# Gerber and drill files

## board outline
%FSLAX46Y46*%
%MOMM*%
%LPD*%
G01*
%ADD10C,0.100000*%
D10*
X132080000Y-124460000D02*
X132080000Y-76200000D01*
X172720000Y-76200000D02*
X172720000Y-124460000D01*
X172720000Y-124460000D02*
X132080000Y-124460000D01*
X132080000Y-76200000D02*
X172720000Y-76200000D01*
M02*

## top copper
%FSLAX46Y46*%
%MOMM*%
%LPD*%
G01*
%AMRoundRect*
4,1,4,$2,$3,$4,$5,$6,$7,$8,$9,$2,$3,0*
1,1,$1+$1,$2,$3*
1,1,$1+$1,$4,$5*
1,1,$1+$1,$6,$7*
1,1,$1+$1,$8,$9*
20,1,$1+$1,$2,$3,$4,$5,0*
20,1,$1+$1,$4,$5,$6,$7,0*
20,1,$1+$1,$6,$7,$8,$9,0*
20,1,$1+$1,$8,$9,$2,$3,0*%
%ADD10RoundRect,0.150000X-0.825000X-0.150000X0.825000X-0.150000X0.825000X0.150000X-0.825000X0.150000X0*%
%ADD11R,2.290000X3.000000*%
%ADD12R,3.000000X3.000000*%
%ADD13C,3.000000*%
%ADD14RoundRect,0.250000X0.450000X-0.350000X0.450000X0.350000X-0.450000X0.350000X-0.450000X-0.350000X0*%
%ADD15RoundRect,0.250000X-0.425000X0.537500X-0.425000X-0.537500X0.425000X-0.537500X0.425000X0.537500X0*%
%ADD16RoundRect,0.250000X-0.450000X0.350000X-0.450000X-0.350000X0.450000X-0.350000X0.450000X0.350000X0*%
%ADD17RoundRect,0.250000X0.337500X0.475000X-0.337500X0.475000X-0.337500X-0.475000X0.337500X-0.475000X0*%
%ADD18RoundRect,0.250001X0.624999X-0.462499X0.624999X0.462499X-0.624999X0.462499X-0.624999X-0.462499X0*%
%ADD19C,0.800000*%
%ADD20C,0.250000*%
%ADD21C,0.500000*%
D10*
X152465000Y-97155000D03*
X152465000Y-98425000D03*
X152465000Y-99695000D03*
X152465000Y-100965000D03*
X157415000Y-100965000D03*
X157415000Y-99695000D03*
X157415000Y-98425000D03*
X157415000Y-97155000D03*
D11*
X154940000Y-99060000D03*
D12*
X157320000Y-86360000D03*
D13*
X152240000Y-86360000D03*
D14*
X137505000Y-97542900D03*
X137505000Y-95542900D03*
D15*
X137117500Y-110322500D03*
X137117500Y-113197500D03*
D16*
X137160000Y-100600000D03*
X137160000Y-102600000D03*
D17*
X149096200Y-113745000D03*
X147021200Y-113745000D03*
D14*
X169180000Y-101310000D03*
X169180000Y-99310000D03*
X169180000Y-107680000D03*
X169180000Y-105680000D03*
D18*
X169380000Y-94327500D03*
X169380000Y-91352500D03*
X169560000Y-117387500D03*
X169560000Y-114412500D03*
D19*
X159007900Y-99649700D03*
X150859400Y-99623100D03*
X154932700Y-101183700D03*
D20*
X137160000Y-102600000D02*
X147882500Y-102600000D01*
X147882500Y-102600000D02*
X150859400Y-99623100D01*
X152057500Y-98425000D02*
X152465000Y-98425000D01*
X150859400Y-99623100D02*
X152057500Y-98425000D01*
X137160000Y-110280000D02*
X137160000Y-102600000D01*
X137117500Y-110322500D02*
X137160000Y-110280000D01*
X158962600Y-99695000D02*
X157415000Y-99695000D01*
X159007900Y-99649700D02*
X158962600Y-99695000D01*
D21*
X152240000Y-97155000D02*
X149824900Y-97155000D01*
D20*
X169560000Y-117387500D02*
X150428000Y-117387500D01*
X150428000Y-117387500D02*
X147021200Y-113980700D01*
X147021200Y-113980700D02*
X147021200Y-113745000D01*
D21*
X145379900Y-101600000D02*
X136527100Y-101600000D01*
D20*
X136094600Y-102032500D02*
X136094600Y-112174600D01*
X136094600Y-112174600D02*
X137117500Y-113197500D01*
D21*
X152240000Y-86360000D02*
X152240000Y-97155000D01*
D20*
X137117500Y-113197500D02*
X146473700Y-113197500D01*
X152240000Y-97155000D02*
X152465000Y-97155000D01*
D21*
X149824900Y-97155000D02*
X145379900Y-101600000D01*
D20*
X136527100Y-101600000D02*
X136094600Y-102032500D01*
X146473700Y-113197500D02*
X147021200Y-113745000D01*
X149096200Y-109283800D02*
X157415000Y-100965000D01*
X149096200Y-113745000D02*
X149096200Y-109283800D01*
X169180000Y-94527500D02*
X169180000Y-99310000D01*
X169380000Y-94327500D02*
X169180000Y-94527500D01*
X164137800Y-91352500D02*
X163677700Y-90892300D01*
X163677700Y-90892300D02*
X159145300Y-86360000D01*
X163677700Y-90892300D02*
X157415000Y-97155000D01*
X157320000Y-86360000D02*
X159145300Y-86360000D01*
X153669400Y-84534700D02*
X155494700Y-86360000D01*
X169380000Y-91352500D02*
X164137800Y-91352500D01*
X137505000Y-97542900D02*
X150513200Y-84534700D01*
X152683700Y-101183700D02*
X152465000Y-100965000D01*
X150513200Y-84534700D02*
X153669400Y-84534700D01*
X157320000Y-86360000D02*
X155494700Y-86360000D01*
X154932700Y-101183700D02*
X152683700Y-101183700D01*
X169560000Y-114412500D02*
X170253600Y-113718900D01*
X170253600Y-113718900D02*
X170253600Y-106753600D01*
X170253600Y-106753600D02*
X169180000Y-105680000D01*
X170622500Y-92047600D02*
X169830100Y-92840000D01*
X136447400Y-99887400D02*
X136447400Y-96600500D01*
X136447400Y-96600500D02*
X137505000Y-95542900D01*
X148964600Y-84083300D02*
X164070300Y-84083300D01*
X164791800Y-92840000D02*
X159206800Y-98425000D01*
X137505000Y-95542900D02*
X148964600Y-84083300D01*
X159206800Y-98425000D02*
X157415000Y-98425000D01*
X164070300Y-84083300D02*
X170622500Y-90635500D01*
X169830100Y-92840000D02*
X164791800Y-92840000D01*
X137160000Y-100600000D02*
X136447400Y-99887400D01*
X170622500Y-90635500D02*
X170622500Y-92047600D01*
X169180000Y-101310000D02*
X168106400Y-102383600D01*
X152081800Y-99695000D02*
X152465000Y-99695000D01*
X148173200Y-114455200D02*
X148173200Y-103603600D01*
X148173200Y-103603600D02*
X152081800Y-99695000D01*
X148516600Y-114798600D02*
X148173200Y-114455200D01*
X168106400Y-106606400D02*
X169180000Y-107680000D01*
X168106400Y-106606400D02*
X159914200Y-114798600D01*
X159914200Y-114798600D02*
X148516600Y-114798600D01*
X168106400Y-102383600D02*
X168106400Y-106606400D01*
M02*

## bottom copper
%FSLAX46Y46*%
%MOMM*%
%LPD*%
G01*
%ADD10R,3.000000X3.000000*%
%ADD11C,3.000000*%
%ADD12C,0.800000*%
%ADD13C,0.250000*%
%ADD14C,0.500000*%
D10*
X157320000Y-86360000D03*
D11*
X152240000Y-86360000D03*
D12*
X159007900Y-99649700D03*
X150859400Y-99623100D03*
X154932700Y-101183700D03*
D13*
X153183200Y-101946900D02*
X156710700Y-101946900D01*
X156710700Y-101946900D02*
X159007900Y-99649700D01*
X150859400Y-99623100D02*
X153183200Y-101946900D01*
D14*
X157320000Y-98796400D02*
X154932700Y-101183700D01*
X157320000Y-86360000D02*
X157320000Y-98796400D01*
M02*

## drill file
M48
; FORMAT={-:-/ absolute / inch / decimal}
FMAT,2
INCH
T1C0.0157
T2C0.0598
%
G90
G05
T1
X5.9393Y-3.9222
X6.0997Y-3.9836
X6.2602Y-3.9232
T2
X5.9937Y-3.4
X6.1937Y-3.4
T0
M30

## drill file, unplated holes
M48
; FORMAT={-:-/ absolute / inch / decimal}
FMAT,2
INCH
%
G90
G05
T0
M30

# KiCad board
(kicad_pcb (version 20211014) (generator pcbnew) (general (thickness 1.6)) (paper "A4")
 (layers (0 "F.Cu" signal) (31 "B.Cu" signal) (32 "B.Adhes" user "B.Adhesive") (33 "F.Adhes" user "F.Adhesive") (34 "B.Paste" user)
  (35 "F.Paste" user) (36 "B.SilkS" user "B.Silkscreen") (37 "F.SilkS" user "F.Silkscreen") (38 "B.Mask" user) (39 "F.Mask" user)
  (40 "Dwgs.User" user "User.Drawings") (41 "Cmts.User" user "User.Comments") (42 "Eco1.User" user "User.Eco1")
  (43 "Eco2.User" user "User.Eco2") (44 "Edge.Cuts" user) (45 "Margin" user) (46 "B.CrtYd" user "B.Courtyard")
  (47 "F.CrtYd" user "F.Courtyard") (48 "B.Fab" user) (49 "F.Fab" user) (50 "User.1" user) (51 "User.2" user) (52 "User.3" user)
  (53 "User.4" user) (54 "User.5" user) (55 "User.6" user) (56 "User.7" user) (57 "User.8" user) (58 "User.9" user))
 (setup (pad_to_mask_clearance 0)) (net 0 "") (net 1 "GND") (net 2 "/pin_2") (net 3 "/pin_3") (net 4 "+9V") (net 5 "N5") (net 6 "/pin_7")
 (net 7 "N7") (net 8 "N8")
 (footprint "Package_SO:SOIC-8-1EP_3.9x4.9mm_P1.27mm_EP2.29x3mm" (layer "F.Cu") (at 154.94 99.06)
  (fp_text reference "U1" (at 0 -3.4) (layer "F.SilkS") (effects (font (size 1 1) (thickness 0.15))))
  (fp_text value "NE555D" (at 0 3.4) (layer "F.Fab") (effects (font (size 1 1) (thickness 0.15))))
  (pad "" smd roundrect (at 0.57 -0.75) (size 0.92 1.21) (layers "F.Paste") (roundrect_rratio 0.25))
  (pad "" smd roundrect (at -0.57 0.75) (size 0.92 1.21) (layers "F.Paste") (roundrect_rratio 0.25))
  (pad "" smd roundrect (at -0.57 -0.75) (size 0.92 1.21) (layers "F.Paste") (roundrect_rratio 0.25))
  (pad "" smd roundrect (at 0.57 0.75) (size 0.92 1.21) (layers "F.Paste") (roundrect_rratio 0.25))
  (pad "1" smd roundrect (at -2.475 -1.905) (size 1.95 0.6) (layers "F.Cu" "F.Paste" "F.Mask") (roundrect_rratio 0.25) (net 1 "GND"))
  (pad "2" smd roundrect (at -2.475 -0.635) (size 1.95 0.6) (layers "F.Cu" "F.Paste" "F.Mask") (roundrect_rratio 0.25) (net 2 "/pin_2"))
  (pad "3" smd roundrect (at -2.475 0.635) (size 1.95 0.6) (layers "F.Cu" "F.Paste" "F.Mask") (roundrect_rratio 0.25) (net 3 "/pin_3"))
  (pad "4" smd roundrect (at -2.475 1.905) (size 1.95 0.6) (layers "F.Cu" "F.Paste" "F.Mask") (roundrect_rratio 0.25) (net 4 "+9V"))
  (pad "5" smd roundrect (at 2.475 1.905) (size 1.95 0.6) (layers "F.Cu" "F.Paste" "F.Mask") (roundrect_rratio 0.25) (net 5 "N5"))
  (pad "6" smd roundrect (at 2.475 0.635) (size 1.95 0.6) (layers "F.Cu" "F.Paste" "F.Mask") (roundrect_rratio 0.25) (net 2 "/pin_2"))
  (pad "7" smd roundrect (at 2.475 -0.635) (size 1.95 0.6) (layers "F.Cu" "F.Paste" "F.Mask") (roundrect_rratio 0.25) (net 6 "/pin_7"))
  (pad "8" smd roundrect (at 2.475 -1.905) (size 1.95 0.6) (layers "F.Cu" "F.Paste" "F.Mask") (roundrect_rratio 0.25) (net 4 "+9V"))
  (pad "9" smd rect (at 0 0) (size 2.29 3) (layers "F.Cu" "F.Mask")))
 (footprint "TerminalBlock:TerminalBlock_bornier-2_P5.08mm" (layer "F.Cu") (at 157.32 86.36 180)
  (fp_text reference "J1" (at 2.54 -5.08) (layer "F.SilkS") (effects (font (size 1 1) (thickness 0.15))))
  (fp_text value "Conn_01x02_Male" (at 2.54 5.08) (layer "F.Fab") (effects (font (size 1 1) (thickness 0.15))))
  (pad "1" thru_hole rect (at 0 0 180) (size 3 3) (drill 1.52) (layers *.Cu *.Mask) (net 4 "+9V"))
  (pad "2" thru_hole circle (at 5.08 0 180) (size 3 3) (drill 1.52) (layers *.Cu *.Mask) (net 1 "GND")))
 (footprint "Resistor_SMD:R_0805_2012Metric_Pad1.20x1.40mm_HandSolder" (layer "F.Cu") (at 137.505 96.5429 90)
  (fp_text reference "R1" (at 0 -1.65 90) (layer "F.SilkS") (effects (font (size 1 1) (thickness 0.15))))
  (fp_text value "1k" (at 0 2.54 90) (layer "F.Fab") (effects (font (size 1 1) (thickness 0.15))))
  (pad "1" smd roundrect (at -1 0 90) (size 1.2 1.4) (layers "F.Cu" "F.Paste" "F.Mask") (roundrect_rratio 0.2083333333) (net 4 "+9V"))
  (pad "2" smd roundrect (at 1 0 90) (size 1.2 1.4) (layers "F.Cu" "F.Paste" "F.Mask") (roundrect_rratio 0.2083333333) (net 6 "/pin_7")))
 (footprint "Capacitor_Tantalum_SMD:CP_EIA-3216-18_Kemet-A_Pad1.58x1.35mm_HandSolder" (layer "F.Cu") (at 137.1175 111.76 -90)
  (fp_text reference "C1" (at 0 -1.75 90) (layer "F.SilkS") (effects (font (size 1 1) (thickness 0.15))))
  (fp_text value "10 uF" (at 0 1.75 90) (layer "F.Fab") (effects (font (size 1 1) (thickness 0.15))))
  (pad "1" smd roundrect (at -1.4375 0 270) (size 1.575 1.35) (layers "F.Cu" "F.Paste" "F.Mask") (roundrect_rratio 0.1851851852)
   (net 2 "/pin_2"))
  (pad "2" smd roundrect (at 1.4375 0 270) (size 1.575 1.35) (layers "F.Cu" "F.Paste" "F.Mask") (roundrect_rratio 0.1851851852)
   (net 1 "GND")))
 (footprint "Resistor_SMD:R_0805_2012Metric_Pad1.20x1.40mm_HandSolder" (layer "F.Cu") (at 137.16 101.6 -90)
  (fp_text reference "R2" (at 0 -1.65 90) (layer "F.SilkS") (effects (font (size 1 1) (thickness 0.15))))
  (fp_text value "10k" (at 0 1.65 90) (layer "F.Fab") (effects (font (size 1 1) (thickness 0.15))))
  (pad "1" smd roundrect (at -1 0 270) (size 1.2 1.4) (layers "F.Cu" "F.Paste" "F.Mask") (roundrect_rratio 0.2083333333) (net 6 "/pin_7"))
  (pad "2" smd roundrect (at 1 0 270) (size 1.2 1.4) (layers "F.Cu" "F.Paste" "F.Mask") (roundrect_rratio 0.2083333333) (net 2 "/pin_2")))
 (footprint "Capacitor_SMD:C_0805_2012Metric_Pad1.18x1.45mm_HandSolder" (layer "F.Cu") (at 148.0587 113.745 180)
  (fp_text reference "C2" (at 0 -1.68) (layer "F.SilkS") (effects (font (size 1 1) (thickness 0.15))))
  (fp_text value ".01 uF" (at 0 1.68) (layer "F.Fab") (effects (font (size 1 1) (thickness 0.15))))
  (pad "1" smd roundrect (at -1.0375 0 180) (size 1.175 1.45) (layers "F.Cu" "F.Paste" "F.Mask") (roundrect_rratio 0.2127659574)
   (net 5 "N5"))
  (pad "2" smd roundrect (at 1.0375 0 180) (size 1.175 1.45) (layers "F.Cu" "F.Paste" "F.Mask") (roundrect_rratio 0.2127659574)
   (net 1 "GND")))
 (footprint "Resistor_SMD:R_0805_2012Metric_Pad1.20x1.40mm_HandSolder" (layer "F.Cu") (at 169.18 100.31 90)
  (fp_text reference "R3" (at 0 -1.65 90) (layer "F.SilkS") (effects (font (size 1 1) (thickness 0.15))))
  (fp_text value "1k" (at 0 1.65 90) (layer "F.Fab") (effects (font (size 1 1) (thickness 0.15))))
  (pad "1" smd roundrect (at -1 0 90) (size 1.2 1.4) (layers "F.Cu" "F.Paste" "F.Mask") (roundrect_rratio 0.2083333333) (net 3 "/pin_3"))
  (pad "2" smd roundrect (at 1 0 90) (size 1.2 1.4) (layers "F.Cu" "F.Paste" "F.Mask") (roundrect_rratio 0.2083333333) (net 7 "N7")))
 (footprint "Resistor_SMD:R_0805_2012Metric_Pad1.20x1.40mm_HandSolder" (layer "F.Cu") (at 169.18 106.68 90)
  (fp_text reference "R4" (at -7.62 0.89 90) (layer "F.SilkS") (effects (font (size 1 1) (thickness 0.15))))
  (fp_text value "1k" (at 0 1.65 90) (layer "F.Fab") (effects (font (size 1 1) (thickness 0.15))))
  (pad "1" smd roundrect (at -1 0 90) (size 1.2 1.4) (layers "F.Cu" "F.Paste" "F.Mask") (roundrect_rratio 0.2083333333) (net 3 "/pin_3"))
  (pad "2" smd roundrect (at 1 0 90) (size 1.2 1.4) (layers "F.Cu" "F.Paste" "F.Mask") (roundrect_rratio 0.2083333333) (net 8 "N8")))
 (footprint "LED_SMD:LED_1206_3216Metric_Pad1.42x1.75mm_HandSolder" (layer "F.Cu") (at 169.38 92.84 90)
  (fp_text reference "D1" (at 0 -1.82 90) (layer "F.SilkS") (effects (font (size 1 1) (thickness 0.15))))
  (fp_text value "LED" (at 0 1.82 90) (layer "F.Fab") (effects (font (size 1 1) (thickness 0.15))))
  (pad "1" smd roundrect (at -1.4875 0 90) (size 1.425 1.75) (layers "F.Cu" "F.Paste" "F.Mask") (roundrect_rratio 0.1754392982) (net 7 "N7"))
  (pad "2" smd roundrect (at 1.4875 0 90) (size 1.425 1.75) (layers "F.Cu" "F.Paste" "F.Mask") (roundrect_rratio 0.1754392982) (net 4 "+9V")))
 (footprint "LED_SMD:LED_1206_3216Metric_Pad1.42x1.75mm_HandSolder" (layer "F.Cu") (at 169.56 115.9 90)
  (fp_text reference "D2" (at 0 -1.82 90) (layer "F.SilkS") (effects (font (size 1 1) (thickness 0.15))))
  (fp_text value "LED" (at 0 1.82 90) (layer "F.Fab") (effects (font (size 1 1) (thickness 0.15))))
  (pad "1" smd roundrect (at -1.4875 0 90) (size 1.425 1.75) (layers "F.Cu" "F.Paste" "F.Mask") (roundrect_rratio 0.1754392982)
   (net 1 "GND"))
  (pad "2" smd roundrect (at 1.4875 0 90) (size 1.425 1.75) (layers "F.Cu" "F.Paste" "F.Mask") (roundrect_rratio 0.1754392982) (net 8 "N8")))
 (gr_line (start 132.08 124.46) (end 132.08 76.2) (layer "Edge.Cuts") (width 0.1))
 (gr_line (start 172.72 76.2) (end 172.72 124.46) (layer "Edge.Cuts") (width 0.1))
 (gr_line (start 172.72 124.46) (end 132.08 124.46) (layer "Edge.Cuts") (width 0.1))
 (gr_line (start 132.08 76.2) (end 172.72 76.2) (layer "Edge.Cuts") (width 0.1))
 (segment (start 137.16 102.6) (end 147.8825 102.6) (width 0.25) (layer "F.Cu") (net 2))
 (segment (start 147.8825 102.6) (end 150.8594 99.6231) (width 0.25) (layer "F.Cu") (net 2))
 (segment (start 152.0575 98.425) (end 152.465 98.425) (width 0.25) (layer "F.Cu") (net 2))
 (segment (start 150.8594 99.6231) (end 152.0575 98.425) (width 0.25) (layer "F.Cu") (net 2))
 (segment (start 137.16 110.28) (end 137.16 102.6) (width 0.25) (layer "F.Cu") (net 2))
 (segment (start 137.1175 110.3225) (end 137.16 110.28) (width 0.25) (layer "F.Cu") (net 2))
 (segment (start 158.9626 99.695) (end 157.415 99.695) (width 0.25) (layer "F.Cu") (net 2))
 (segment (start 159.0079 99.6497) (end 158.9626 99.695) (width 0.25) (layer "F.Cu") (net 2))
 (via (at 159.0079 99.6497) (size 0.8) (drill 0.4) (layers "F.Cu" "B.Cu") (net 2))
 (via (at 150.8594 99.6231) (size 0.8) (drill 0.4) (layers "F.Cu" "B.Cu") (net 2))
 (segment (start 153.1832 101.9469) (end 156.7107 101.9469) (width 0.25) (layer "B.Cu") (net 2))
 (segment (start 156.7107 101.9469) (end 159.0079 99.6497) (width 0.25) (layer "B.Cu") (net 2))
 (segment (start 150.8594 99.6231) (end 153.1832 101.9469) (width 0.25) (layer "B.Cu") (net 2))
 (segment (start 152.24 97.155) (end 149.8249 97.155) (width 0.5) (layer "F.Cu") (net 1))
 (segment (start 169.56 117.3875) (end 150.428 117.3875) (width 0.25) (layer "F.Cu") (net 1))
 (segment (start 150.428 117.3875) (end 147.0212 113.9807) (width 0.25) (layer "F.Cu") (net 1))
 (segment (start 147.0212 113.9807) (end 147.0212 113.745) (width 0.25) (layer "F.Cu") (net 1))
 (segment (start 145.3799 101.6) (end 136.5271 101.6) (width 0.5) (layer "F.Cu") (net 1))
 (segment (start 136.0946 102.0325) (end 136.0946 112.1746) (width 0.25) (layer "F.Cu") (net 1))
 (segment (start 136.0946 112.1746) (end 137.1175 113.1975) (width 0.25) (layer "F.Cu") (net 1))
 (segment (start 152.24 86.36) (end 152.24 97.155) (width 0.5) (layer "F.Cu") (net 1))
 (segment (start 137.1175 113.1975) (end 146.4737 113.1975) (width 0.25) (layer "F.Cu") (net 1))
 (segment (start 152.24 97.155) (end 152.465 97.155) (width 0.25) (layer "F.Cu") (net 1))
 (segment (start 149.8249 97.155) (end 145.3799 101.6) (width 0.5) (layer "F.Cu") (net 1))
 (segment (start 136.5271 101.6) (end 136.0946 102.0325) (width 0.25) (layer "F.Cu") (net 1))
 (segment (start 146.4737 113.1975) (end 147.0212 113.745) (width 0.25) (layer "F.Cu") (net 1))
 (segment (start 149.0962 109.2838) (end 157.415 100.965) (width 0.25) (layer "F.Cu") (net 5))
 (segment (start 149.0962 113.745) (end 149.0962 109.2838) (width 0.25) (layer "F.Cu") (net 5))
 (segment (start 169.18 94.5275) (end 169.18 99.31) (width 0.25) (layer "F.Cu") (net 7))
 (segment (start 169.38 94.3275) (end 169.18 94.5275) (width 0.25) (layer "F.Cu") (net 7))
 (segment (start 164.1378 91.3525) (end 163.6777 90.8923) (width 0.25) (layer "F.Cu") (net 4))
 (segment (start 163.6777 90.8923) (end 159.1453 86.36) (width 0.25) (layer "F.Cu") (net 4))
 (segment (start 163.6777 90.8923) (end 157.415 97.155) (width 0.25) (layer "F.Cu") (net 4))
 (segment (start 157.32 86.36) (end 159.1453 86.36) (width 0.25) (layer "F.Cu") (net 4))
 (segment (start 153.6694 84.5347) (end 155.4947 86.36) (width 0.25) (layer "F.Cu") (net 4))
 (segment (start 169.38 91.3525) (end 164.1378 91.3525) (width 0.25) (layer "F.Cu") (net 4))
 (segment (start 137.505 97.5429) (end 150.5132 84.5347) (width 0.25) (layer "F.Cu") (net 4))
 (segment (start 152.6837 101.1837) (end 152.465 100.965) (width 0.25) (layer "F.Cu") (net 4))
 (segment (start 150.5132 84.5347) (end 153.6694 84.5347) (width 0.25) (layer "F.Cu") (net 4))
 (segment (start 157.32 86.36) (end 155.4947 86.36) (width 0.25) (layer "F.Cu") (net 4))
 (segment (start 154.9327 101.1837) (end 152.6837 101.1837) (width 0.25) (layer "F.Cu") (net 4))
 (via (at 154.9327 101.1837) (size 0.8) (drill 0.4) (layers "F.Cu" "B.Cu") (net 4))
 (segment (start 157.32 98.7964) (end 154.9327 101.1837) (width 0.5) (layer "B.Cu") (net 4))
 (segment (start 157.32 86.36) (end 157.32 98.7964) (width 0.5) (layer "B.Cu") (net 4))
 (segment (start 169.56 114.4125) (end 170.2536 113.7189) (width 0.25) (layer "F.Cu") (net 8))
 (segment (start 170.2536 113.7189) (end 170.2536 106.7536) (width 0.25) (layer "F.Cu") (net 8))
 (segment (start 170.2536 106.7536) (end 169.18 105.68) (width 0.25) (layer "F.Cu") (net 8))
 (segment (start 170.6225 92.0476) (end 169.8301 92.84) (width 0.25) (layer "F.Cu") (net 6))
 (segment (start 136.4474 99.8874) (end 136.4474 96.6005) (width 0.25) (layer "F.Cu") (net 6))
 (segment (start 136.4474 96.6005) (end 137.505 95.5429) (width 0.25) (layer "F.Cu") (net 6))
 (segment (start 148.9646 84.0833) (end 164.0703 84.0833) (width 0.25) (layer "F.Cu") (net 6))
 (segment (start 164.7918 92.84) (end 159.2068 98.425) (width 0.25) (layer "F.Cu") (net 6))
 (segment (start 137.505 95.5429) (end 148.9646 84.0833) (width 0.25) (layer "F.Cu") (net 6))
 (segment (start 159.2068 98.425) (end 157.415 98.425) (width 0.25) (layer "F.Cu") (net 6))
 (segment (start 164.0703 84.0833) (end 170.6225 90.6355) (width 0.25) (layer "F.Cu") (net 6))
 (segment (start 169.8301 92.84) (end 164.7918 92.84) (width 0.25) (layer "F.Cu") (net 6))
 (segment (start 137.16 100.6) (end 136.4474 99.8874) (width 0.25) (layer "F.Cu") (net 6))
 (segment (start 170.6225 90.6355) (end 170.6225 92.0476) (width 0.25) (layer "F.Cu") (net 6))
 (segment (start 169.18 101.31) (end 168.1064 102.3836) (width 0.25) (layer "F.Cu") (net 3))
 (segment (start 152.0818 99.695) (end 152.465 99.695) (width 0.25) (layer "F.Cu") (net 3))
 (segment (start 148.1732 114.4552) (end 148.1732 103.6036) (width 0.25) (layer "F.Cu") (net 3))
 (segment (start 148.1732 103.6036) (end 152.0818 99.695) (width 0.25) (layer "F.Cu") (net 3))
 (segment (start 148.5166 114.7986) (end 148.1732 114.4552) (width 0.25) (layer "F.Cu") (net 3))
 (segment (start 168.1064 106.6064) (end 169.18 107.68) (width 0.25) (layer "F.Cu") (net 3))
 (segment (start 168.1064 106.6064) (end 159.9142 114.7986) (width 0.25) (layer "F.Cu") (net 3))
 (segment (start 159.9142 114.7986) (end 148.5166 114.7986) (width 0.25) (layer "F.Cu") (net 3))
 (segment (start 168.1064 102.3836) (end 168.1064 106.6064) (width 0.25) (layer "F.Cu") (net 3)))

